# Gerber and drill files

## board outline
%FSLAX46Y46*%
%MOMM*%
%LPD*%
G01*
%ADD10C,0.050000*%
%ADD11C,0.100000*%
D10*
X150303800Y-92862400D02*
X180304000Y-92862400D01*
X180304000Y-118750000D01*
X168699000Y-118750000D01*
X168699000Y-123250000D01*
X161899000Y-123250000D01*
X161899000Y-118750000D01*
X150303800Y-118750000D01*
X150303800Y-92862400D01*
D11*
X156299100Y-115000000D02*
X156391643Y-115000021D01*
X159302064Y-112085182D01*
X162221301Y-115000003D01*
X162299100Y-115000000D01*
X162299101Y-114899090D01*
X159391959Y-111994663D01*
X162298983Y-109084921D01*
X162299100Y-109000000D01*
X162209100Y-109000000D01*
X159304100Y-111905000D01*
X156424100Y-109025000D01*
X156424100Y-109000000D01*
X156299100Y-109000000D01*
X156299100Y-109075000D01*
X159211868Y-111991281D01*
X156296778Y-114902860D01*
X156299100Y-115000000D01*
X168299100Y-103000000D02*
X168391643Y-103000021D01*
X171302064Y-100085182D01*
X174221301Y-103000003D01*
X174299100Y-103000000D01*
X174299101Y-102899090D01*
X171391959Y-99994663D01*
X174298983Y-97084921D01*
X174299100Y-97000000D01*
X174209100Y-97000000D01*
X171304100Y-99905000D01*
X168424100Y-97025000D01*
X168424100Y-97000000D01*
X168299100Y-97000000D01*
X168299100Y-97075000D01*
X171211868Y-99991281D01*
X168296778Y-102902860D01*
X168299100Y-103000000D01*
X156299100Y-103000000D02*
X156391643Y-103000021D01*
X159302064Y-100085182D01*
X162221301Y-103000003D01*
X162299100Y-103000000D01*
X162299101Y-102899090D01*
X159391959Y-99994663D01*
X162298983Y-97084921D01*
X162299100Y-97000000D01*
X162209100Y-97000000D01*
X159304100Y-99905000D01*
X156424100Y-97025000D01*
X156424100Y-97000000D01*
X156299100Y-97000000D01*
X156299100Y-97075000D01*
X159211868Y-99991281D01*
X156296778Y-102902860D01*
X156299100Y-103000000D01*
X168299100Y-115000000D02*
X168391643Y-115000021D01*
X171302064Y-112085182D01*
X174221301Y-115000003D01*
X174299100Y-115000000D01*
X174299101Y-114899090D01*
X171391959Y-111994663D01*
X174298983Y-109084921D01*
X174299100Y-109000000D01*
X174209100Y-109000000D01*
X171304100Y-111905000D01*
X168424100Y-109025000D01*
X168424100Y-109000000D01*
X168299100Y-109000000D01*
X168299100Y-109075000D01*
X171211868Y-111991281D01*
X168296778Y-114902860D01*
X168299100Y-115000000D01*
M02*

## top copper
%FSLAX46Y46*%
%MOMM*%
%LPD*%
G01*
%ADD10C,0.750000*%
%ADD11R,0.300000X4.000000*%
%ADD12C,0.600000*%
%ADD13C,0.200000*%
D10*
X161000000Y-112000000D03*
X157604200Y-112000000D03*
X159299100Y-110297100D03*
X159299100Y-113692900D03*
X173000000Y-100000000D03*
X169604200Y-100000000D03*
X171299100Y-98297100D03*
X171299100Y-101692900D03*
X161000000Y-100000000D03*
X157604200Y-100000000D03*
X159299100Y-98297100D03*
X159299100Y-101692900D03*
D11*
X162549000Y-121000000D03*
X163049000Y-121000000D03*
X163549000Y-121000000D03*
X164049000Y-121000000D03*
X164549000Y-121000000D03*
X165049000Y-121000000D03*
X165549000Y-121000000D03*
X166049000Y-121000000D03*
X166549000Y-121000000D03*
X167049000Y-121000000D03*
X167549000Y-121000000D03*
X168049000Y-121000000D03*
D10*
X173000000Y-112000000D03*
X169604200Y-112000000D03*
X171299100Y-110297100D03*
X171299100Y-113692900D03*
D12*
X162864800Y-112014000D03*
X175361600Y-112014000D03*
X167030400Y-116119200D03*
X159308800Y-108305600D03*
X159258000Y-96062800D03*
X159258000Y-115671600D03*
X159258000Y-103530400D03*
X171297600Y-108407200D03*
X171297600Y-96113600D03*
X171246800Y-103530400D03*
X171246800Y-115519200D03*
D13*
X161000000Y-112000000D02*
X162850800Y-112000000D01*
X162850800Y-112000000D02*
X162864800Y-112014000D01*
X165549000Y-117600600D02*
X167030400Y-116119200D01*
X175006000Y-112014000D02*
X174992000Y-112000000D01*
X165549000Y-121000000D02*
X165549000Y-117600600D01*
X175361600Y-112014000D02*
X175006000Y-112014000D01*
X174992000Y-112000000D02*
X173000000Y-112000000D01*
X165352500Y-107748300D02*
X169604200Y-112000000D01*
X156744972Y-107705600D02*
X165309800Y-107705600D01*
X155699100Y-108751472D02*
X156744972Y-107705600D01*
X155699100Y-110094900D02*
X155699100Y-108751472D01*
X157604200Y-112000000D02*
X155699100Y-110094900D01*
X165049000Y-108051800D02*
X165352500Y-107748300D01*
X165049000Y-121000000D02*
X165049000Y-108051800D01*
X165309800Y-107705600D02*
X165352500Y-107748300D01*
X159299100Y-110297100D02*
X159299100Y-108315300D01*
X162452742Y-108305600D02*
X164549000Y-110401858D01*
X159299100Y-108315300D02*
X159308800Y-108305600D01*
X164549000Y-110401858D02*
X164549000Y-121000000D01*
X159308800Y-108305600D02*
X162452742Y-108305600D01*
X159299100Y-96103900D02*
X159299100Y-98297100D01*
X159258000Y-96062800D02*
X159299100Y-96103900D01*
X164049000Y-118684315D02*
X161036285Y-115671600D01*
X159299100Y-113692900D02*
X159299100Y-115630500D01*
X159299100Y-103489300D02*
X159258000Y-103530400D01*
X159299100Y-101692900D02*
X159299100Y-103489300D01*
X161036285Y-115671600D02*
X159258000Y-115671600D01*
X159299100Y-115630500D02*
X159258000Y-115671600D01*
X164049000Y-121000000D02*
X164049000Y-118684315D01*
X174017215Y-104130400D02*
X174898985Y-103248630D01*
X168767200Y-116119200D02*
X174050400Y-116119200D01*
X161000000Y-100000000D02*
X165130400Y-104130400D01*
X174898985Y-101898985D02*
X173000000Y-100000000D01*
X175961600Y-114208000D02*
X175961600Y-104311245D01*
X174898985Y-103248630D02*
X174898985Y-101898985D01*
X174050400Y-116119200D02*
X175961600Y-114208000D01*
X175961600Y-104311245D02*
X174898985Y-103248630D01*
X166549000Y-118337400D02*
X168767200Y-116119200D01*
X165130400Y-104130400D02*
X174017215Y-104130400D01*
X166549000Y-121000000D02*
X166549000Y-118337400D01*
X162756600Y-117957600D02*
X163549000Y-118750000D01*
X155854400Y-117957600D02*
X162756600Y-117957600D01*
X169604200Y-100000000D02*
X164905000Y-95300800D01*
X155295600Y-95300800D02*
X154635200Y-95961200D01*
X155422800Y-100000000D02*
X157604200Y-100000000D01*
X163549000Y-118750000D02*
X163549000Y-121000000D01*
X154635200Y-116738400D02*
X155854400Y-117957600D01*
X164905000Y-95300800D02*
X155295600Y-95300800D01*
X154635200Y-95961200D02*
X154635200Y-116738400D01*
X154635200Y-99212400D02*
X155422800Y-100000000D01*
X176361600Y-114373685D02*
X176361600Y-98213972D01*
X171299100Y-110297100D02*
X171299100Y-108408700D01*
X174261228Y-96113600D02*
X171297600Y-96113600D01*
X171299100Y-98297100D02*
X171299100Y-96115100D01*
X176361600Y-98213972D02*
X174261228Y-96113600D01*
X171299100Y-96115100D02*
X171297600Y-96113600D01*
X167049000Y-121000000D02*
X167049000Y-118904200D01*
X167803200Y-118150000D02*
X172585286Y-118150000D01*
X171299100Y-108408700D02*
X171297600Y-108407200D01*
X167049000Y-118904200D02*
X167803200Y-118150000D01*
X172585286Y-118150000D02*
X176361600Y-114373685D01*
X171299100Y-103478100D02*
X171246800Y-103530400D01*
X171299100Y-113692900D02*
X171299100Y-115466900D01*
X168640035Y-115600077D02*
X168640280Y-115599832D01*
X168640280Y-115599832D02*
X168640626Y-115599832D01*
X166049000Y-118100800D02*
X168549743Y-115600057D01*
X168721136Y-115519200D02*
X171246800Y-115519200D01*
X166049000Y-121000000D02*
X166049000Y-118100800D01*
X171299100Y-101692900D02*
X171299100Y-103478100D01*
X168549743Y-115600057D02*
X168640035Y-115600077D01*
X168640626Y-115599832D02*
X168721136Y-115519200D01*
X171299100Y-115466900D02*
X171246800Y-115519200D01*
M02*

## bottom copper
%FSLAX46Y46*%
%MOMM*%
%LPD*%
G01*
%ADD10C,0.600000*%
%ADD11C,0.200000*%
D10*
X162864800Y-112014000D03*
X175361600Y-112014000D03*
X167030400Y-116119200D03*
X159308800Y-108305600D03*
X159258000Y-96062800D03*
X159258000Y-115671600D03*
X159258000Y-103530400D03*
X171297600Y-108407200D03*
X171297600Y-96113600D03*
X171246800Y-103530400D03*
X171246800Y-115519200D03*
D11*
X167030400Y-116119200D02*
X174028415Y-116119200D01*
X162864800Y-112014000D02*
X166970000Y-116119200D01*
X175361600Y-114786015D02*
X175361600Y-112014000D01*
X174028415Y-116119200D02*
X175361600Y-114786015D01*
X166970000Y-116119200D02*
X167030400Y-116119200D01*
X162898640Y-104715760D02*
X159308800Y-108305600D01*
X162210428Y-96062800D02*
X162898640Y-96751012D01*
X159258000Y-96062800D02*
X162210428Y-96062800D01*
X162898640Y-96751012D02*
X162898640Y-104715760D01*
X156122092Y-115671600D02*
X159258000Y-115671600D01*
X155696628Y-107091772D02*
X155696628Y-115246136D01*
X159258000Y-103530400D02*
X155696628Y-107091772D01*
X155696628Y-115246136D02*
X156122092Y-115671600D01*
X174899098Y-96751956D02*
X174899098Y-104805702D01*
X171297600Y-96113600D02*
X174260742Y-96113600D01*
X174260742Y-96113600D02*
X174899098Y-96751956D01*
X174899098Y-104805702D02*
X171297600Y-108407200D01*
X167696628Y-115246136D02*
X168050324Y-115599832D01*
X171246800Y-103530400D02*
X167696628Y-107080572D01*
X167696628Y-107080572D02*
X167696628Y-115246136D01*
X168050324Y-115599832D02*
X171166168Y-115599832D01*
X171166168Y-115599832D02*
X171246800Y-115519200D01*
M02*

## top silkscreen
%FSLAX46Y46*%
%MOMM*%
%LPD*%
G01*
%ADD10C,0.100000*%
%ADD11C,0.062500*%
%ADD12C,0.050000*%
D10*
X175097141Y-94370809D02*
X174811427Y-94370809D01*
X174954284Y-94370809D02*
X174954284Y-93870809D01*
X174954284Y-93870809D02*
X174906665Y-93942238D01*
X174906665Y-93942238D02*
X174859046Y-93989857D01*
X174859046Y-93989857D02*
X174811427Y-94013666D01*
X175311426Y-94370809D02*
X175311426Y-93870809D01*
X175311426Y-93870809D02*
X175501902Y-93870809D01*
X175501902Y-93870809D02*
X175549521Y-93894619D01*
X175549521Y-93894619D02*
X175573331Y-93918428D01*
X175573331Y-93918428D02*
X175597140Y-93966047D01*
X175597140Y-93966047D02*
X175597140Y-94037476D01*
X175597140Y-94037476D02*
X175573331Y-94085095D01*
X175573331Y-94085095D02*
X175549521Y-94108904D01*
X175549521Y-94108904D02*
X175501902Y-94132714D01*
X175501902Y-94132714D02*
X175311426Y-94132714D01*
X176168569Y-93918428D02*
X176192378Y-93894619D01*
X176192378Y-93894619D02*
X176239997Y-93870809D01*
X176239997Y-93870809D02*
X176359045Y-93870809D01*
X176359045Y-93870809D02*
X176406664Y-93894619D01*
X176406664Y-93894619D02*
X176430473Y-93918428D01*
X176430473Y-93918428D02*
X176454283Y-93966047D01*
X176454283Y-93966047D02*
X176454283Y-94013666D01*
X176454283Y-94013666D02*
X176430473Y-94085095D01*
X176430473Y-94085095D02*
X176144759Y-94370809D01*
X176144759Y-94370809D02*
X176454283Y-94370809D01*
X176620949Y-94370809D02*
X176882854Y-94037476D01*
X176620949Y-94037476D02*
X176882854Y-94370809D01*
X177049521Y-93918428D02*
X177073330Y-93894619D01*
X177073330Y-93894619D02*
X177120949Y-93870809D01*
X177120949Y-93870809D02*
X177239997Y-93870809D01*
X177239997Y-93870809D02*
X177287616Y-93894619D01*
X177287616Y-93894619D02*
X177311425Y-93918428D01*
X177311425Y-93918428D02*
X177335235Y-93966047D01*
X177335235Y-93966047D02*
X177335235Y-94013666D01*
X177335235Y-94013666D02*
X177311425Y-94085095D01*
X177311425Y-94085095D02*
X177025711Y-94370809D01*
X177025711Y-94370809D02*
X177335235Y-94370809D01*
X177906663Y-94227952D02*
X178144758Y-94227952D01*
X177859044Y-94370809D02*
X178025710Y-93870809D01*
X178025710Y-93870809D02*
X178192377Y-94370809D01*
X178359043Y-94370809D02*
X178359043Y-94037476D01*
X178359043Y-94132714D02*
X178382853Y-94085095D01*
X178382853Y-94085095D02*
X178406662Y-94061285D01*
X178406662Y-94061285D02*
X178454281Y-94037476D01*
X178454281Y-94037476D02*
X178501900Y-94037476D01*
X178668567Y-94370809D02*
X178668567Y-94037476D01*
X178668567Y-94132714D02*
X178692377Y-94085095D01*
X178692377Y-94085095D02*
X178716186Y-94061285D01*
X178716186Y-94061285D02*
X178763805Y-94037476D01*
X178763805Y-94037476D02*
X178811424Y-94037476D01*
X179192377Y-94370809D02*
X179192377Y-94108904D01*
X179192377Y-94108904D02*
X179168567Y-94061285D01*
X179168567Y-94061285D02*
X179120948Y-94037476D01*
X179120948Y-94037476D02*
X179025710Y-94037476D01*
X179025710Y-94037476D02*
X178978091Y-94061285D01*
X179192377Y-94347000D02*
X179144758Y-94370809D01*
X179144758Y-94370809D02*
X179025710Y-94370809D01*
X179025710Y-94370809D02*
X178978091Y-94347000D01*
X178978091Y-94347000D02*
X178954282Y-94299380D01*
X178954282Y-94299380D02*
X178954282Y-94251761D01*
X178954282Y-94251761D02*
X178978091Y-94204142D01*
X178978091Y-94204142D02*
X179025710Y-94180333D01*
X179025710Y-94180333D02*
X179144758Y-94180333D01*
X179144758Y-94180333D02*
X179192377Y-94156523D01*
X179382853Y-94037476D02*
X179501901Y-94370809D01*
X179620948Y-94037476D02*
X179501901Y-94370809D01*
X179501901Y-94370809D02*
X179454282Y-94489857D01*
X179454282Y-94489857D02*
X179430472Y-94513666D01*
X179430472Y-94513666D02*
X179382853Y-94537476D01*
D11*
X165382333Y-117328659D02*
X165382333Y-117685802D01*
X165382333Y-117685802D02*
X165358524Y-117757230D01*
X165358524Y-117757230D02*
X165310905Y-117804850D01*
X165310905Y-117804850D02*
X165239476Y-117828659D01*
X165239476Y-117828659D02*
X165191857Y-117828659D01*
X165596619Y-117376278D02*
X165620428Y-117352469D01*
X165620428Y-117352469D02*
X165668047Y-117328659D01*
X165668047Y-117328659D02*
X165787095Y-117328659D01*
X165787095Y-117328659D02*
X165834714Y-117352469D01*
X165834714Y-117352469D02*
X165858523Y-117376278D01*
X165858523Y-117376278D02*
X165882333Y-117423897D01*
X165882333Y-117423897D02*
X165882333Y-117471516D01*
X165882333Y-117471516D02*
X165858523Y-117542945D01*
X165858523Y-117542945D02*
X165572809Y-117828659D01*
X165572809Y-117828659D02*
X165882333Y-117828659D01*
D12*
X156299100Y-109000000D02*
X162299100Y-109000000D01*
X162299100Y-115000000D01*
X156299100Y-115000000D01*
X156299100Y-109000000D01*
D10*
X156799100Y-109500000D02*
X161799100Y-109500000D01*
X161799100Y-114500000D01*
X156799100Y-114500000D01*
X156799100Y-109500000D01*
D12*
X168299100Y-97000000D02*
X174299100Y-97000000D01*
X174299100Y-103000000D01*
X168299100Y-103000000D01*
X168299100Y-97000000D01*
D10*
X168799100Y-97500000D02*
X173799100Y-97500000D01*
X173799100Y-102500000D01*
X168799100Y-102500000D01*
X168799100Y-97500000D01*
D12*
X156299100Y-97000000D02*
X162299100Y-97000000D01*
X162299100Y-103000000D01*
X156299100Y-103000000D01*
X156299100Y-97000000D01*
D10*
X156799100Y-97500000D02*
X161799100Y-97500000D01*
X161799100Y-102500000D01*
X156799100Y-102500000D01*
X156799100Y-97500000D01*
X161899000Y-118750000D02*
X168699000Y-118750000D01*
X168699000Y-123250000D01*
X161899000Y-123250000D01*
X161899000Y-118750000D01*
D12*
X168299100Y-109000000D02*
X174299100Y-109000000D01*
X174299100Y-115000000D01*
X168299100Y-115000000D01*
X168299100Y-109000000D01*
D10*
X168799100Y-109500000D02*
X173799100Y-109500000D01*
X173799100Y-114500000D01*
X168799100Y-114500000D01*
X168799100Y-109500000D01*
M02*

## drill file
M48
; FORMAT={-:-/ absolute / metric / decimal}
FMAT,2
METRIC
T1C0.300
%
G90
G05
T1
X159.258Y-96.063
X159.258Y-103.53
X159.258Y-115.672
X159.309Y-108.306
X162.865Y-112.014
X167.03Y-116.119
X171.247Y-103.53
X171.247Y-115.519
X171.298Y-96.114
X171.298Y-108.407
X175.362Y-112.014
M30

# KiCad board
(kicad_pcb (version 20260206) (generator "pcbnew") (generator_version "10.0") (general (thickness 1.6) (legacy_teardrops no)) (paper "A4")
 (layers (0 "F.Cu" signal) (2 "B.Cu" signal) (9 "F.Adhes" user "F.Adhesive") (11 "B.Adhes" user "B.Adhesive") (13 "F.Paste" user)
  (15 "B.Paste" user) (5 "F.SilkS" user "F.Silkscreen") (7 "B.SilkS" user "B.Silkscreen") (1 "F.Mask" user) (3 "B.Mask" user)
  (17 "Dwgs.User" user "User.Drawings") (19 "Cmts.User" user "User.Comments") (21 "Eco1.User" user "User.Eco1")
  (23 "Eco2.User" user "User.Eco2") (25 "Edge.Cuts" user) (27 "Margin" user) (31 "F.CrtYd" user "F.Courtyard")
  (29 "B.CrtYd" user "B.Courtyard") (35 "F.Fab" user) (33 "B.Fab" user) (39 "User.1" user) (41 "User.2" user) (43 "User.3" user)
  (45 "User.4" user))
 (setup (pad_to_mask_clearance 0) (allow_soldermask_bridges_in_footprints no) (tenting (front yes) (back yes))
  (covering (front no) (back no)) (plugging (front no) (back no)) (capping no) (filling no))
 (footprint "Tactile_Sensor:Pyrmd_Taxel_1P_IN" (layer "F.Cu") (at 159.2991 112)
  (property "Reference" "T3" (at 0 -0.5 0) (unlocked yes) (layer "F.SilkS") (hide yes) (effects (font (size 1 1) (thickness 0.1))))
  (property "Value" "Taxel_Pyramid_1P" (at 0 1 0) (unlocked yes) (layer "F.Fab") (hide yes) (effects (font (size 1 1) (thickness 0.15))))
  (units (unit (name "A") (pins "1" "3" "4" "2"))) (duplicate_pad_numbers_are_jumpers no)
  (fp_rect (start -3 -3) (end 3 3) (stroke (width 0.05) (type solid)) (fill no) (layer "F.SilkS"))
  (fp_rect (start -2.5 -2.5) (end 2.5 2.5) (stroke (width 0.1) (type solid)) (fill no) (layer "F.SilkS"))
  (fp_poly
   (pts (xy -3 3) (xy -2.907457 3.000021) (xy 0.002964 0.085182) (xy 2.922201 3.000003) (xy 3 3) (xy 3.000001 2.89909)
    (xy 0.092859 -0.005337) (xy 2.999883 -2.915079) (xy 3 -3) (xy 2.91 -3) (xy 0.005 -0.095) (xy -2.875 -2.975) (xy -2.875 -3) (xy -3 -3)
    (xy -3 -2.925) (xy -0.087232 -0.008719) (xy -3.002322 2.90286))
   (stroke (width 0.1) (type solid)) (fill no) (layer "Edge.Cuts"))
  (pad "1" smd circle (at 1.7009 0 90) (size 0.75 0.75) (layers "F.Cu" "F.Mask" "F.Paste") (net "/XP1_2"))
  (pad "2" smd circle (at -1.6949 0 270) (size 0.75 0.75) (layers "F.Cu" "F.Mask") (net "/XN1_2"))
  (pad "3" smd circle (at 0 -1.7029) (size 0.75 0.75) (layers "F.Cu" "F.Mask") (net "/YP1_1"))
  (pad "4" smd circle (at 0 1.6929) (size 0.75 0.75) (layers "F.Cu" "F.Mask") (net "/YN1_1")))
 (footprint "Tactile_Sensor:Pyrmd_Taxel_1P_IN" (layer "F.Cu") (at 171.2991 100)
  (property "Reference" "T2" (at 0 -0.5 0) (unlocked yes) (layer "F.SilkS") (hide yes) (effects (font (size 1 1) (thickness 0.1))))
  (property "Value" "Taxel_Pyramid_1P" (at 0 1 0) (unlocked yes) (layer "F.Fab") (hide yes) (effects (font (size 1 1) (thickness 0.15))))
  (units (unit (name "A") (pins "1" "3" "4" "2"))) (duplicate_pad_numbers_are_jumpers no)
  (fp_rect (start -3 -3) (end 3 3) (stroke (width 0.05) (type solid)) (fill no) (layer "F.SilkS"))
  (fp_rect (start -2.5 -2.5) (end 2.5 2.5) (stroke (width 0.1) (type solid)) (fill no) (layer "F.SilkS"))
  (fp_poly
   (pts (xy -3 3) (xy -2.907457 3.000021) (xy 0.002964 0.085182) (xy 2.922201 3.000003) (xy 3 3) (xy 3.000001 2.89909)
    (xy 0.092859 -0.005337) (xy 2.999883 -2.915079) (xy 3 -3) (xy 2.91 -3) (xy 0.005 -0.095) (xy -2.875 -2.975) (xy -2.875 -3) (xy -3 -3)
    (xy -3 -2.925) (xy -0.087232 -0.008719) (xy -3.002322 2.90286))
   (stroke (width 0.1) (type solid)) (fill no) (layer "Edge.Cuts"))
  (pad "1" smd circle (at 1.7009 0 90) (size 0.75 0.75) (layers "F.Cu" "F.Mask" "F.Paste") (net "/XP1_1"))
  (pad "2" smd circle (at -1.6949 0 270) (size 0.75 0.75) (layers "F.Cu" "F.Mask") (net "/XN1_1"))
  (pad "3" smd circle (at 0 -1.7029) (size 0.75 0.75) (layers "F.Cu" "F.Mask") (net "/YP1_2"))
  (pad "4" smd circle (at 0 1.6929) (size 0.75 0.75) (layers "F.Cu" "F.Mask") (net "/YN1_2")))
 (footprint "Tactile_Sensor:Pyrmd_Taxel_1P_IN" (layer "F.Cu") (at 159.2991 100)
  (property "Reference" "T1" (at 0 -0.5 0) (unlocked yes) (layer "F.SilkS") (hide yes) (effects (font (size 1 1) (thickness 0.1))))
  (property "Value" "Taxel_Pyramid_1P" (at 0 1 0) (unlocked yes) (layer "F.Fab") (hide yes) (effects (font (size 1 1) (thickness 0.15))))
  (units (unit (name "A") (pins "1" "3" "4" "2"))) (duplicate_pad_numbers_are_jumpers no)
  (fp_rect (start -3 -3) (end 3 3) (stroke (width 0.05) (type solid)) (fill no) (layer "F.SilkS"))
  (fp_rect (start -2.5 -2.5) (end 2.5 2.5) (stroke (width 0.1) (type solid)) (fill no) (layer "F.SilkS"))
  (fp_poly
   (pts (xy -3 3) (xy -2.907457 3.000021) (xy 0.002964 0.085182) (xy 2.922201 3.000003) (xy 3 3) (xy 3.000001 2.89909)
    (xy 0.092859 -0.005337) (xy 2.999883 -2.915079) (xy 3 -3) (xy 2.91 -3) (xy 0.005 -0.095) (xy -2.875 -2.975) (xy -2.875 -3) (xy -3 -3)
    (xy -3 -2.925) (xy -0.087232 -0.008719) (xy -3.002322 2.90286))
   (stroke (width 0.1) (type solid)) (fill no) (layer "Edge.Cuts"))
  (pad "1" smd circle (at 1.7009 0 90) (size 0.75 0.75) (layers "F.Cu" "F.Mask" "F.Paste") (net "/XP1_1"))
  (pad "2" smd circle (at -1.6949 0 270) (size 0.75 0.75) (layers "F.Cu" "F.Mask") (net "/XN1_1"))
  (pad "3" smd circle (at 0 -1.7029) (size 0.75 0.75) (layers "F.Cu" "F.Mask") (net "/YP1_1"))
  (pad "4" smd circle (at 0 1.6929) (size 0.75 0.75) (layers "F.Cu" "F.Mask") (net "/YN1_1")))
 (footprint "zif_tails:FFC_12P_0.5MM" (layer "F.Cu") (at 165.439 119)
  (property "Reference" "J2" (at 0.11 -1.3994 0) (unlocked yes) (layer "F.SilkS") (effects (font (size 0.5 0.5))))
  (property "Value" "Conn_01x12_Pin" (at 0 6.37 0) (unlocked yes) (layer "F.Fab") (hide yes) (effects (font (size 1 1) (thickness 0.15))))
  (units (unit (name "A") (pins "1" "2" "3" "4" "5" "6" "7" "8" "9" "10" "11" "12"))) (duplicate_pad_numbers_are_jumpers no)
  (fp_rect (start -3.54 -0.25) (end 3.26 4.25) (stroke (width 0.1) (type default)) (fill no) (layer "F.SilkS"))
  (pad "1" smd rect (at -2.89 2) (size 0.3 4) (layers "F.Cu" "F.Mask") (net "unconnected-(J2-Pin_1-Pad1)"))
  (pad "2" smd rect (at -2.39 2) (size 0.3 4) (layers "F.Cu" "F.Mask") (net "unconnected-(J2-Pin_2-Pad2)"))
  (pad "3" smd rect (at -1.89 2) (size 0.3 4) (layers "F.Cu" "F.Mask") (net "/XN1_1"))
  (pad "4" smd rect (at -1.39 2) (size 0.3 4) (layers "F.Cu" "F.Mask") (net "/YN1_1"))
  (pad "5" smd rect (at -0.89 2) (size 0.3 4) (layers "F.Cu" "F.Mask") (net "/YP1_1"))
  (pad "6" smd rect (at -0.39 2) (size 0.3 4) (layers "F.Cu" "F.Mask") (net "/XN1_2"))
  (pad "7" smd rect (at 0.11 2) (size 0.3 4) (layers "F.Cu" "F.Mask") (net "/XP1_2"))
  (pad "8" smd rect (at 0.61 2) (size 0.3 4) (layers "F.Cu" "F.Mask") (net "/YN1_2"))
  (pad "9" smd rect (at 1.11 2) (size 0.3 4) (layers "F.Cu" "F.Mask") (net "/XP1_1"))
  (pad "10" smd rect (at 1.61 2) (size 0.3 4) (layers "F.Cu" "F.Mask") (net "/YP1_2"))
  (pad "11" smd rect (at 2.11 2) (size 0.3 4) (layers "F.Cu" "F.Mask") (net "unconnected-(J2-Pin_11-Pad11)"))
  (pad "12" smd rect (at 2.61 2) (size 0.3 4) (layers "F.Cu" "F.Mask") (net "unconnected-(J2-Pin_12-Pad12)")))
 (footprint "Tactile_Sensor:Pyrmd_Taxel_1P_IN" (layer "F.Cu") (at 171.2991 112)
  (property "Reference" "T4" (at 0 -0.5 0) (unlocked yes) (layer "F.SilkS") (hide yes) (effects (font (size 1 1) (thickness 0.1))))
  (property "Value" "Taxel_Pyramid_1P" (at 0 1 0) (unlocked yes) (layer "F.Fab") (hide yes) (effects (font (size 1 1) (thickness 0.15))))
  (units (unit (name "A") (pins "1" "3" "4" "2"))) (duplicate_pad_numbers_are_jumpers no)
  (fp_rect (start -3 -3) (end 3 3) (stroke (width 0.05) (type solid)) (fill no) (layer "F.SilkS"))
  (fp_rect (start -2.5 -2.5) (end 2.5 2.5) (stroke (width 0.1) (type solid)) (fill no) (layer "F.SilkS"))
  (fp_poly
   (pts (xy -3 3) (xy -2.907457 3.000021) (xy 0.002964 0.085182) (xy 2.922201 3.000003) (xy 3 3) (xy 3.000001 2.89909)
    (xy 0.092859 -0.005337) (xy 2.999883 -2.915079) (xy 3 -3) (xy 2.91 -3) (xy 0.005 -0.095) (xy -2.875 -2.975) (xy -2.875 -3) (xy -3 -3)
    (xy -3 -2.925) (xy -0.087232 -0.008719) (xy -3.002322 2.90286))
   (stroke (width 0.1) (type solid)) (fill no) (layer "Edge.Cuts"))
  (pad "1" smd circle (at 1.7009 0 90) (size 0.75 0.75) (layers "F.Cu" "F.Mask" "F.Paste") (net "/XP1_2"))
  (pad "2" smd circle (at -1.6949 0 270) (size 0.75 0.75) (layers "F.Cu" "F.Mask") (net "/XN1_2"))
  (pad "3" smd circle (at 0 -1.7029) (size 0.75 0.75) (layers "F.Cu" "F.Mask") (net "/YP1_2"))
  (pad "4" smd circle (at 0 1.6929) (size 0.75 0.75) (layers "F.Cu" "F.Mask") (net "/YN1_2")))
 (gr_poly
  (pts (xy 150.3038 92.8624) (xy 180.304 92.8624) (xy 180.304 118.75) (xy 168.699 118.75) (xy 168.699 123.25) (xy 161.899 123.25)
   (xy 161.899 118.75) (xy 150.3038 118.75))
  (stroke (width 0.05) (type solid)) (fill no) (layer "Edge.Cuts"))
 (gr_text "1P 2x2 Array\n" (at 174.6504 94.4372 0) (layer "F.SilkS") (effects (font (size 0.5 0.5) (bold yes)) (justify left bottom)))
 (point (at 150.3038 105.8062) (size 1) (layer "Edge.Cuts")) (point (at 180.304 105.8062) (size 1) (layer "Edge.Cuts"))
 (segment (start 161 112) (end 162.8508 112) (width 0.2) (layer "F.Cu") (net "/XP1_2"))
 (segment (start 162.8508 112) (end 162.8648 112.014) (width 0.2) (layer "F.Cu") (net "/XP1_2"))
 (segment (start 165.549 117.6006) (end 167.0304 116.1192) (width 0.2) (layer "F.Cu") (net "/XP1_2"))
 (segment (start 175.006 112.014) (end 174.992 112) (width 0.2) (layer "F.Cu") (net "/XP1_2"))
 (segment (start 165.549 121) (end 165.549 117.6006) (width 0.2) (layer "F.Cu") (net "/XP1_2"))
 (segment (start 175.3616 112.014) (end 175.006 112.014) (width 0.2) (layer "F.Cu") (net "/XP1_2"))
 (segment (start 174.992 112) (end 173 112) (width 0.2) (layer "F.Cu") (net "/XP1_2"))
 (via (at 162.8648 112.014) (size 0.6) (drill 0.3) (layers "F.Cu" "B.Cu") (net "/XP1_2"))
 (via (at 175.3616 112.014) (size 0.6) (drill 0.3) (layers "F.Cu" "B.Cu") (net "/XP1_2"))
 (via (at 167.0304 116.1192) (size 0.6) (drill 0.3) (layers "F.Cu" "B.Cu") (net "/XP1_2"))
 (segment (start 167.0304 116.1192) (end 174.028415 116.1192) (width 0.2) (layer "B.Cu") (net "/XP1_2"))
 (segment (start 162.8648 112.014) (end 166.97 116.1192) (width 0.2) (layer "B.Cu") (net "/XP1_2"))
 (segment (start 175.3616 114.786015) (end 175.3616 112.014) (width 0.2) (layer "B.Cu") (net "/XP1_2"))
 (segment (start 174.028415 116.1192) (end 175.3616 114.786015) (width 0.2) (layer "B.Cu") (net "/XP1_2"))
 (segment (start 166.97 116.1192) (end 167.0304 116.1192) (width 0.2) (layer "B.Cu") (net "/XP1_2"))
 (segment (start 165.3525 107.7483) (end 169.6042 112) (width 0.2) (layer "F.Cu") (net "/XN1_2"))
 (segment (start 156.744972 107.7056) (end 165.3098 107.7056) (width 0.2) (layer "F.Cu") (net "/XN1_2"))
 (segment (start 155.6991 108.751472) (end 156.744972 107.7056) (width 0.2) (layer "F.Cu") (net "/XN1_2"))
 (segment (start 155.6991 110.0949) (end 155.6991 108.751472) (width 0.2) (layer "F.Cu") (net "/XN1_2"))
 (segment (start 157.6042 112) (end 155.6991 110.0949) (width 0.2) (layer "F.Cu") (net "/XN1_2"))
 (segment (start 165.049 108.0518) (end 165.3525 107.7483) (width 0.2) (layer "F.Cu") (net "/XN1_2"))
 (segment (start 165.049 121) (end 165.049 108.0518) (width 0.2) (layer "F.Cu") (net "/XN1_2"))
 (segment (start 165.3098 107.7056) (end 165.3525 107.7483) (width 0.2) (layer "F.Cu") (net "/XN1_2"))
 (segment (start 159.2991 110.2971) (end 159.2991 108.3153) (width 0.2) (layer "F.Cu") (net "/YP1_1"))
 (segment (start 162.452742 108.3056) (end 164.549 110.401858) (width 0.2) (layer "F.Cu") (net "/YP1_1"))
 (segment (start 159.2991 108.3153) (end 159.3088 108.3056) (width 0.2) (layer "F.Cu") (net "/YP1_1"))
 (segment (start 164.549 110.401858) (end 164.549 121) (width 0.2) (layer "F.Cu") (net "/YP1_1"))
 (segment (start 159.3088 108.3056) (end 162.452742 108.3056) (width 0.2) (layer "F.Cu") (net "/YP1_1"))
 (segment (start 159.2991 96.1039) (end 159.2991 98.2971) (width 0.2) (layer "F.Cu") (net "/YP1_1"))
 (segment (start 159.258 96.0628) (end 159.2991 96.1039) (width 0.2) (layer "F.Cu") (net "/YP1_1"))
 (via (at 159.3088 108.3056) (size 0.6) (drill 0.3) (layers "F.Cu" "B.Cu") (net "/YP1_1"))
 (via (at 159.258 96.0628) (size 0.6) (drill 0.3) (layers "F.Cu" "B.Cu") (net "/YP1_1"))
 (segment (start 162.89864 104.71576) (end 159.3088 108.3056) (width 0.2) (layer "B.Cu") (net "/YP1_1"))
 (segment (start 162.210428 96.0628) (end 162.89864 96.751012) (width 0.2) (layer "B.Cu") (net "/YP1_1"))
 (segment (start 159.258 96.0628) (end 162.210428 96.0628) (width 0.2) (layer "B.Cu") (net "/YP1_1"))
 (segment (start 162.89864 96.751012) (end 162.89864 104.71576) (width 0.2) (layer "B.Cu") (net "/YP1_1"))
 (segment (start 164.049 118.684315) (end 161.036285 115.6716) (width 0.2) (layer "F.Cu") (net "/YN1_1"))
 (segment (start 159.2991 113.6929) (end 159.2991 115.6305) (width 0.2) (layer "F.Cu") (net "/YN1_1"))
 (segment (start 159.2991 103.4893) (end 159.258 103.5304) (width 0.2) (layer "F.Cu") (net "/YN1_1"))
 (segment (start 159.2991 101.6929) (end 159.2991 103.4893) (width 0.2) (layer "F.Cu") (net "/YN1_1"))
 (segment (start 161.036285 115.6716) (end 159.258 115.6716) (width 0.2) (layer "F.Cu") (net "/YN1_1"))
 (segment (start 159.2991 115.6305) (end 159.258 115.6716) (width 0.2) (layer "F.Cu") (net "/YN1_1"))
 (segment (start 164.049 121) (end 164.049 118.684315) (width 0.2) (layer "F.Cu") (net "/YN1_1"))
 (via (at 159.258 115.6716) (size 0.6) (drill 0.3) (layers "F.Cu" "B.Cu") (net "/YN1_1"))
 (via (at 159.258 103.5304) (size 0.6) (drill 0.3) (layers "F.Cu" "B.Cu") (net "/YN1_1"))
 (segment (start 156.122092 115.6716) (end 159.258 115.6716) (width 0.2) (layer "B.Cu") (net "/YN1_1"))
 (segment (start 155.696628 107.091772) (end 155.696628 115.246136) (width 0.2) (layer "B.Cu") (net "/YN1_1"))
 (segment (start 159.258 103.5304) (end 155.696628 107.091772) (width 0.2) (layer "B.Cu") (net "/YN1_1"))
 (segment (start 155.696628 115.246136) (end 156.122092 115.6716) (width 0.2) (layer "B.Cu") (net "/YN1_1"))
 (segment (start 174.017215 104.1304) (end 174.898985 103.24863) (width 0.2) (layer "F.Cu") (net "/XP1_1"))
 (segment (start 168.7672 116.1192) (end 174.0504 116.1192) (width 0.2) (layer "F.Cu") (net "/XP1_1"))
 (segment (start 161 100) (end 165.1304 104.1304) (width 0.2) (layer "F.Cu") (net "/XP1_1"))
 (segment (start 174.898985 101.898985) (end 173 100) (width 0.2) (layer "F.Cu") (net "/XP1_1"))
 (segment (start 175.9616 114.208) (end 175.9616 104.311245) (width 0.2) (layer "F.Cu") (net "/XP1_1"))
 (segment (start 174.898985 103.24863) (end 174.898985 101.898985) (width 0.2) (layer "F.Cu") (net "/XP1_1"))
 (segment (start 174.0504 116.1192) (end 175.9616 114.208) (width 0.2) (layer "F.Cu") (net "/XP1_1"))
 (segment (start 175.9616 104.311245) (end 174.898985 103.24863) (width 0.2) (layer "F.Cu") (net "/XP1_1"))
 (segment (start 166.549 118.3374) (end 168.7672 116.1192) (width 0.2) (layer "F.Cu") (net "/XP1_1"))
 (segment (start 165.1304 104.1304) (end 174.017215 104.1304) (width 0.2) (layer "F.Cu") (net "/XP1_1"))
 (segment (start 166.549 121) (end 166.549 118.3374) (width 0.2) (layer "F.Cu") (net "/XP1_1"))
 (segment (start 162.7566 117.9576) (end 163.549 118.75) (width 0.2) (layer "F.Cu") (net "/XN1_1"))
 (segment (start 155.8544 117.9576) (end 162.7566 117.9576) (width 0.2) (layer "F.Cu") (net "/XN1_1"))
 (segment (start 169.6042 100) (end 164.905 95.3008) (width 0.2) (layer "F.Cu") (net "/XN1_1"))
 (segment (start 155.2956 95.3008) (end 154.6352 95.9612) (width 0.2) (layer "F.Cu") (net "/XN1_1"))
 (segment (start 155.4228 100) (end 157.6042 100) (width 0.2) (layer "F.Cu") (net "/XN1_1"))
 (segment (start 163.549 118.75) (end 163.549 121) (width 0.2) (layer "F.Cu") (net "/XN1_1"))
 (segment (start 154.6352 116.7384) (end 155.8544 117.9576) (width 0.2) (layer "F.Cu") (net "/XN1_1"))
 (segment (start 164.905 95.3008) (end 155.2956 95.3008) (width 0.2) (layer "F.Cu") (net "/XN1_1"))
 (segment (start 154.6352 95.9612) (end 154.6352 116.7384) (width 0.2) (layer "F.Cu") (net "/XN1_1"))
 (segment (start 154.6352 99.2124) (end 155.4228 100) (width 0.2) (layer "F.Cu") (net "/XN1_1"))
 (segment (start 176.3616 114.373685) (end 176.3616 98.213972) (width 0.2) (layer "F.Cu") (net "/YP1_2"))
 (segment (start 171.2991 110.2971) (end 171.2991 108.4087) (width 0.2) (layer "F.Cu") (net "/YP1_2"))
 (segment (start 174.261228 96.1136) (end 171.2976 96.1136) (width 0.2) (layer "F.Cu") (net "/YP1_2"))
 (segment (start 171.2991 98.2971) (end 171.2991 96.1151) (width 0.2) (layer "F.Cu") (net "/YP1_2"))
 (segment (start 176.3616 98.213972) (end 174.261228 96.1136) (width 0.2) (layer "F.Cu") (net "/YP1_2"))
 (segment (start 171.2991 96.1151) (end 171.2976 96.1136) (width 0.2) (layer "F.Cu") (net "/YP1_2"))
 (segment (start 167.049 121) (end 167.049 118.9042) (width 0.2) (layer "F.Cu") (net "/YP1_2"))
 (segment (start 167.8032 118.15) (end 172.585286 118.15) (width 0.2) (layer "F.Cu") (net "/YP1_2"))
 (segment (start 171.2991 108.4087) (end 171.2976 108.4072) (width 0.2) (layer "F.Cu") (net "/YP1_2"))
 (segment (start 167.049 118.9042) (end 167.8032 118.15) (width 0.2) (layer "F.Cu") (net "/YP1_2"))
 (segment (start 172.585286 118.15) (end 176.3616 114.373685) (width 0.2) (layer "F.Cu") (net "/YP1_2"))
 (via (at 171.2976 108.4072) (size 0.6) (drill 0.3) (layers "F.Cu" "B.Cu") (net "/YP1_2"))
 (via (at 171.2976 96.1136) (size 0.6) (drill 0.3) (layers "F.Cu" "B.Cu") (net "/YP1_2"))
 (segment (start 174.899098 96.751956) (end 174.899098 104.805702) (width 0.2) (layer "B.Cu") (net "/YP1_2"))
 (segment (start 171.2976 96.1136) (end 174.260742 96.1136) (width 0.2) (layer "B.Cu") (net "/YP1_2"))
 (segment (start 174.260742 96.1136) (end 174.899098 96.751956) (width 0.2) (layer "B.Cu") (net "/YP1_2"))
 (segment (start 174.899098 104.805702) (end 171.2976 108.4072) (width 0.2) (layer "B.Cu") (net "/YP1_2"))
 (segment (start 171.2991 103.4781) (end 171.2468 103.5304) (width 0.2) (layer "F.Cu") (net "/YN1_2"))
 (segment (start 171.2991 113.6929) (end 171.2991 115.4669) (width 0.2) (layer "F.Cu") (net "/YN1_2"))
 (segment (start 168.640035 115.600077) (end 168.64028 115.599832) (width 0.2) (layer "F.Cu") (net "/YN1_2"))
 (segment (start 168.64028 115.599832) (end 168.640626 115.599832) (width 0.2) (layer "F.Cu") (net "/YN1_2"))
 (segment (start 166.049 118.1008) (end 168.549743 115.600057) (width 0.2) (layer "F.Cu") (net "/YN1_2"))
 (segment (start 168.721136 115.5192) (end 171.2468 115.5192) (width 0.2) (layer "F.Cu") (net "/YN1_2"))
 (segment (start 166.049 121) (end 166.049 118.1008) (width 0.2) (layer "F.Cu") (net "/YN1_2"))
 (segment (start 171.2991 101.6929) (end 171.2991 103.4781) (width 0.2) (layer "F.Cu") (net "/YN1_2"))
 (segment (start 168.549743 115.600057) (end 168.640035 115.600077) (width 0.2) (layer "F.Cu") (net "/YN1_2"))
 (segment (start 168.640626 115.599832) (end 168.721136 115.5192) (width 0.2) (layer "F.Cu") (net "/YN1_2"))
 (segment (start 171.2991 115.4669) (end 171.2468 115.5192) (width 0.2) (layer "F.Cu") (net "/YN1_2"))
 (via (at 171.2468 103.5304) (size 0.6) (drill 0.3) (layers "F.Cu" "B.Cu") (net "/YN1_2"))
 (via (at 171.2468 115.5192) (size 0.6) (drill 0.3) (layers "F.Cu" "B.Cu") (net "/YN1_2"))
 (segment (start 167.696628 115.246136) (end 168.050324 115.599832) (width 0.2) (layer "B.Cu") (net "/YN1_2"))
 (segment (start 171.2468 103.5304) (end 167.696628 107.080572) (width 0.2) (layer "B.Cu") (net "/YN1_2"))
 (segment (start 167.696628 107.080572) (end 167.696628 115.246136) (width 0.2) (layer "B.Cu") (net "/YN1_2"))
 (segment (start 168.050324 115.599832) (end 171.166168 115.599832) (width 0.2) (layer "B.Cu") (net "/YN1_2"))
 (segment (start 171.166168 115.599832) (end 171.2468 115.5192) (width 0.2) (layer "B.Cu") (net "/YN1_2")))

